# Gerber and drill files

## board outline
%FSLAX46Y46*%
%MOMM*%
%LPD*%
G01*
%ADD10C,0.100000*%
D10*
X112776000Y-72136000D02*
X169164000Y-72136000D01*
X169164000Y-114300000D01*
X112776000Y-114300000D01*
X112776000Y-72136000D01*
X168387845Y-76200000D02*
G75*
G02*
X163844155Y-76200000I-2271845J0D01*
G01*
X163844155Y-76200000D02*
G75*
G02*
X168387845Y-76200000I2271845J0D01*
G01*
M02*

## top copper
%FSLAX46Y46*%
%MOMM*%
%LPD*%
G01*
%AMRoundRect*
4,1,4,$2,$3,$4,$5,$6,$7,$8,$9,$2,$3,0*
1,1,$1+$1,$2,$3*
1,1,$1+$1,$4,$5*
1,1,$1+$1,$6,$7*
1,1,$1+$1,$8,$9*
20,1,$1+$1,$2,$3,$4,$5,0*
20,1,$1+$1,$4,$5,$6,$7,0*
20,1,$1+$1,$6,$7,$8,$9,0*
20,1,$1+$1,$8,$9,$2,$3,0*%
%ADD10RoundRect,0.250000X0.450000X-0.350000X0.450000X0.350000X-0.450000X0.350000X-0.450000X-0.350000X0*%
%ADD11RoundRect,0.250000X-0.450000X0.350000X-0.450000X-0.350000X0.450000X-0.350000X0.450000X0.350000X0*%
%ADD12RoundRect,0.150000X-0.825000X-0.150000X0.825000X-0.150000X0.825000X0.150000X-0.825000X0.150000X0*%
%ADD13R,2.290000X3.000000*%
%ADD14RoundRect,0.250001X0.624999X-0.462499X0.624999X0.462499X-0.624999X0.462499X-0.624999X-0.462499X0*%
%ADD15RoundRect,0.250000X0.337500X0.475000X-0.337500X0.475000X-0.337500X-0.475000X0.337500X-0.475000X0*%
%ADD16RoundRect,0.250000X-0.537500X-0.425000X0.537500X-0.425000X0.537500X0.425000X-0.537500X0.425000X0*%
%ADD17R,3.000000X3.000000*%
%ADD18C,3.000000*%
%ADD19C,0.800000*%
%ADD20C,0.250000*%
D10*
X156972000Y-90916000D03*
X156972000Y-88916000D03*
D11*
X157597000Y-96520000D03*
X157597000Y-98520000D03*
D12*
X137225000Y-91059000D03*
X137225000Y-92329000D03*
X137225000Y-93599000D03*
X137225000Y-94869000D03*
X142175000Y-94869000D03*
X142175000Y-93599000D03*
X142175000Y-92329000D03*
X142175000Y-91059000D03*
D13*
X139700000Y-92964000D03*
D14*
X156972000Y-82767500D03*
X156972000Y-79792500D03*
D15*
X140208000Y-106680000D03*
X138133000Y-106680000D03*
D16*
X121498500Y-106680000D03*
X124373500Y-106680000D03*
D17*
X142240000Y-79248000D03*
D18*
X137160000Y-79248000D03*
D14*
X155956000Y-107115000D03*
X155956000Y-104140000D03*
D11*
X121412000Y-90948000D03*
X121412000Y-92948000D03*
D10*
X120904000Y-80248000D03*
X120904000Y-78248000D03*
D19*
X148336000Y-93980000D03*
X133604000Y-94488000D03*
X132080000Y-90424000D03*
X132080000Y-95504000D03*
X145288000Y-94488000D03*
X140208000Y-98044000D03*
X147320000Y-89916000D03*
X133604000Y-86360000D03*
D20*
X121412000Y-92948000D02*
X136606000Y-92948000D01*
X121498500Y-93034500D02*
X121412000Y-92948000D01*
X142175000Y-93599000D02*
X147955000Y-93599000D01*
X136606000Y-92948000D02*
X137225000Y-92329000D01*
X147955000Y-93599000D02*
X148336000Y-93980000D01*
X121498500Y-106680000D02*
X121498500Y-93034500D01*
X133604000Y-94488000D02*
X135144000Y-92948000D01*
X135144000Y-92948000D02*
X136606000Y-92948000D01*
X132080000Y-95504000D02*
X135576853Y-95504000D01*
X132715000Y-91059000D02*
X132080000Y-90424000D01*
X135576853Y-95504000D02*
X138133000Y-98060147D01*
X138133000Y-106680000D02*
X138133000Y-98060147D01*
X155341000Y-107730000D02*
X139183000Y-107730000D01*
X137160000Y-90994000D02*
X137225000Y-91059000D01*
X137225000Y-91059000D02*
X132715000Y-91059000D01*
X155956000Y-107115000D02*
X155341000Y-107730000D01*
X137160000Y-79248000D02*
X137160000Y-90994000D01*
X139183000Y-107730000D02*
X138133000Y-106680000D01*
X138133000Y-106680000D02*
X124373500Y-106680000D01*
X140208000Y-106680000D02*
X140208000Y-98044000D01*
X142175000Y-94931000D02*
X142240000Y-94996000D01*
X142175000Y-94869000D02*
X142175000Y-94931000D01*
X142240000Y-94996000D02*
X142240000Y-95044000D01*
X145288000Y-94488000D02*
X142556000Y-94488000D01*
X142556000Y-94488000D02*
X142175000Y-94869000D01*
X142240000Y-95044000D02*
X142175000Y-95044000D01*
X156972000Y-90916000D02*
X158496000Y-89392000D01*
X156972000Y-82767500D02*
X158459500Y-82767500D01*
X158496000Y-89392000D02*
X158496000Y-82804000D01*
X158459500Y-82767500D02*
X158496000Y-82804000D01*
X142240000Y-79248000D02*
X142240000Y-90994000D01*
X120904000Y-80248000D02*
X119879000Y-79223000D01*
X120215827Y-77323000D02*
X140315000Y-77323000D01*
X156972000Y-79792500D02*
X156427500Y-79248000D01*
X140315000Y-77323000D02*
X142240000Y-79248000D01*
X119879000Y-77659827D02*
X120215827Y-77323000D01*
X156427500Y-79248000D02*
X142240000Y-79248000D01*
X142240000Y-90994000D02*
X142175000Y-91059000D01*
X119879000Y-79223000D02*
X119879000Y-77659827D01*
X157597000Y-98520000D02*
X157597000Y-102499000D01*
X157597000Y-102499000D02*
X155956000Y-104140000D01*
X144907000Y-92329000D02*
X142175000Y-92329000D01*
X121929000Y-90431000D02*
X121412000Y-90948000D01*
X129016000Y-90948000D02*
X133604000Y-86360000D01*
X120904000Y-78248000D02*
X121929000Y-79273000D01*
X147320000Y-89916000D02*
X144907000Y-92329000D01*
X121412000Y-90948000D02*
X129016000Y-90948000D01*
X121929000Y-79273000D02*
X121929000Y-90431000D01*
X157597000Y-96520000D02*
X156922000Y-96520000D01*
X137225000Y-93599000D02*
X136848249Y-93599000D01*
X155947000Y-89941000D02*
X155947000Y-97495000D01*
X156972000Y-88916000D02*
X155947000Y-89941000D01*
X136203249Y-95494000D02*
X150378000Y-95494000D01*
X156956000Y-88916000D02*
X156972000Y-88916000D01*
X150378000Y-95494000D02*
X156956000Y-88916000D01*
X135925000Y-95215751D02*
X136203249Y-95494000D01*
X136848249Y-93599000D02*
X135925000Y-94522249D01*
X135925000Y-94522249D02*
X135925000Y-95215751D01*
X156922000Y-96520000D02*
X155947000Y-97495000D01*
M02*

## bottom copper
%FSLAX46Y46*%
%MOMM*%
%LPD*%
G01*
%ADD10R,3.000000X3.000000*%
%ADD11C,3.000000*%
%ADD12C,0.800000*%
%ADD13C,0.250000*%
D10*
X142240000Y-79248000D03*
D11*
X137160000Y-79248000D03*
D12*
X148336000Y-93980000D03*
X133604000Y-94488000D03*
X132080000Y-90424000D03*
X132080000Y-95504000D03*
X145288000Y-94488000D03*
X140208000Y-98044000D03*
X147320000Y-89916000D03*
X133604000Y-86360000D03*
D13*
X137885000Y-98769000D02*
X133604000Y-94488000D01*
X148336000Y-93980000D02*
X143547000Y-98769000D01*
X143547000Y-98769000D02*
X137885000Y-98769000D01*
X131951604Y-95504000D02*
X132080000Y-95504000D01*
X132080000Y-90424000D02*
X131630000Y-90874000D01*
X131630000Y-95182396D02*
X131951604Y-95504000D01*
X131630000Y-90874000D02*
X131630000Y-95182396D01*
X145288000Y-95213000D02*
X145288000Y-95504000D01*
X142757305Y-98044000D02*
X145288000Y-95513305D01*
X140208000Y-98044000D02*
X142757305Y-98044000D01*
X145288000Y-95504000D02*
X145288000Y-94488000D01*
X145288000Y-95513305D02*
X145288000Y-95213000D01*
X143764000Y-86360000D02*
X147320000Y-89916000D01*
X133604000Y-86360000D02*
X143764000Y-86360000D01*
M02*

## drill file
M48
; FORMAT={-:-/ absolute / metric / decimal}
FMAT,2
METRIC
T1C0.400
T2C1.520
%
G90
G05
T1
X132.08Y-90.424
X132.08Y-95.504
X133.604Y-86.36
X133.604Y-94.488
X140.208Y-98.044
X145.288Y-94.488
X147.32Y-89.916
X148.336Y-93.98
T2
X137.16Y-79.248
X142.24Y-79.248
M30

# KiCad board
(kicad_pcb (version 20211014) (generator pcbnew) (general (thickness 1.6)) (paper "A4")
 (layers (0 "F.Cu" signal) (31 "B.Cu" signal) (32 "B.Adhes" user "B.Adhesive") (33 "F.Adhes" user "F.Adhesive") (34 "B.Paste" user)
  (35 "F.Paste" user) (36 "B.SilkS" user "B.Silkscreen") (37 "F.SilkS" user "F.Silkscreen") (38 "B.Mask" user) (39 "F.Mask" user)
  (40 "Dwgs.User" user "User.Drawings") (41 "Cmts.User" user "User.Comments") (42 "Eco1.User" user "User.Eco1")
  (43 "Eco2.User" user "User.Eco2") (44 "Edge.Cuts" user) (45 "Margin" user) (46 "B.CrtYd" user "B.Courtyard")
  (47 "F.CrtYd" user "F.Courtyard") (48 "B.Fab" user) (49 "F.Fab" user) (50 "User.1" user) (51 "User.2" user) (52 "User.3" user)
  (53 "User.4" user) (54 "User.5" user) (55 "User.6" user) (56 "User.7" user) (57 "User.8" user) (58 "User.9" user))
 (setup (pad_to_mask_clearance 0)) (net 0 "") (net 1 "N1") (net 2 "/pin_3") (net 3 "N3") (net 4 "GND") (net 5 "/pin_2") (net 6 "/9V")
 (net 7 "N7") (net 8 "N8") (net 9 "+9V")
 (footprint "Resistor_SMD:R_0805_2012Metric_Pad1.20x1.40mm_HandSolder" (layer "F.Cu") (at 156.972 89.916 90)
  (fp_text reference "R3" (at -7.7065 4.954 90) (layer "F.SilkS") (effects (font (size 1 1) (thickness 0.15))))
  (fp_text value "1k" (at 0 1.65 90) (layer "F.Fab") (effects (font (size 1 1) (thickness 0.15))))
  (pad "1" smd roundrect (at -1 0 90) (size 1.2 1.4) (layers "F.Cu" "F.Paste" "F.Mask") (roundrect_rratio 0.208333) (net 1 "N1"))
  (pad "2" smd roundrect (at 1 0 90) (size 1.2 1.4) (layers "F.Cu" "F.Paste" "F.Mask") (roundrect_rratio 0.208333) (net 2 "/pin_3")))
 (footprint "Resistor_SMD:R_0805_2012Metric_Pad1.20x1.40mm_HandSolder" (layer "F.Cu") (at 157.597 97.52 -90)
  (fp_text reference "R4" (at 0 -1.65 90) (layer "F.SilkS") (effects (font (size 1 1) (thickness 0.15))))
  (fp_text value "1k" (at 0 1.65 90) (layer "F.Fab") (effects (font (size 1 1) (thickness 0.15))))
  (pad "1" smd roundrect (at -1 0 270) (size 1.2 1.4) (layers "F.Cu" "F.Paste" "F.Mask") (roundrect_rratio 0.208333) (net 2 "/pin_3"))
  (pad "2" smd roundrect (at 1 0 270) (size 1.2 1.4) (layers "F.Cu" "F.Paste" "F.Mask") (roundrect_rratio 0.208333) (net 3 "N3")))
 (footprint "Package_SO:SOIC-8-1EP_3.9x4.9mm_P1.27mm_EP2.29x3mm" (layer "F.Cu") (at 139.7 92.964)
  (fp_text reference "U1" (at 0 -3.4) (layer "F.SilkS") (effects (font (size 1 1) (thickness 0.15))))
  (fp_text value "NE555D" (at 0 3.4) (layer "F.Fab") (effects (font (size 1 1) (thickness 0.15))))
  (pad "" smd roundrect (at 0.57 -0.75) (size 0.92 1.21) (layers "F.Paste") (roundrect_rratio 0.25))
  (pad "" smd roundrect (at -0.57 0.75) (size 0.92 1.21) (layers "F.Paste") (roundrect_rratio 0.25))
  (pad "" smd roundrect (at -0.57 -0.75) (size 0.92 1.21) (layers "F.Paste") (roundrect_rratio 0.25))
  (pad "" smd roundrect (at 0.57 0.75) (size 0.92 1.21) (layers "F.Paste") (roundrect_rratio 0.25))
  (pad "1" smd roundrect (at -2.475 -1.905) (size 1.95 0.6) (layers "F.Cu" "F.Paste" "F.Mask") (roundrect_rratio 0.25) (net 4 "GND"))
  (pad "2" smd roundrect (at -2.475 -0.635) (size 1.95 0.6) (layers "F.Cu" "F.Paste" "F.Mask") (roundrect_rratio 0.25) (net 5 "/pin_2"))
  (pad "3" smd roundrect (at -2.475 0.635) (size 1.95 0.6) (layers "F.Cu" "F.Paste" "F.Mask") (roundrect_rratio 0.25) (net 2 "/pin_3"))
  (pad "4" smd roundrect (at -2.475 1.905) (size 1.95 0.6) (layers "F.Cu" "F.Paste" "F.Mask") (roundrect_rratio 0.25) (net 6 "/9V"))
  (pad "5" smd roundrect (at 2.475 1.905) (size 1.95 0.6) (layers "F.Cu" "F.Paste" "F.Mask") (roundrect_rratio 0.25) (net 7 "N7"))
  (pad "6" smd roundrect (at 2.475 0.635) (size 1.95 0.6) (layers "F.Cu" "F.Paste" "F.Mask") (roundrect_rratio 0.25) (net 5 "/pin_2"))
  (pad "7" smd roundrect (at 2.475 -0.635) (size 1.95 0.6) (layers "F.Cu" "F.Paste" "F.Mask") (roundrect_rratio 0.25) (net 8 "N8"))
  (pad "8" smd roundrect (at 2.475 -1.905) (size 1.95 0.6) (layers "F.Cu" "F.Paste" "F.Mask") (roundrect_rratio 0.25) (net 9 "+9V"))
  (pad "9" smd rect (at 0 0) (size 2.29 3) (layers "F.Cu" "F.Mask")))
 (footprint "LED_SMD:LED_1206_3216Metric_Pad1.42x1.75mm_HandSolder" (layer "F.Cu") (at 156.972 81.28 90)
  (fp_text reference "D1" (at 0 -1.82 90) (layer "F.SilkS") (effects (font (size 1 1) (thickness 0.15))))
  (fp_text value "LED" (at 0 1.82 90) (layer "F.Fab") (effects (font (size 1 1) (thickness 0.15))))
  (pad "1" smd roundrect (at -1.4875 0 90) (size 1.425 1.75) (layers "F.Cu" "F.Paste" "F.Mask") (roundrect_rratio 0.175439) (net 1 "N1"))
  (pad "2" smd roundrect (at 1.4875 0 90) (size 1.425 1.75) (layers "F.Cu" "F.Paste" "F.Mask") (roundrect_rratio 0.175439) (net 9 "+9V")))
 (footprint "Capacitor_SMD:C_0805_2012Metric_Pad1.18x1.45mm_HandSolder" (layer "F.Cu") (at 139.1705 106.68 180)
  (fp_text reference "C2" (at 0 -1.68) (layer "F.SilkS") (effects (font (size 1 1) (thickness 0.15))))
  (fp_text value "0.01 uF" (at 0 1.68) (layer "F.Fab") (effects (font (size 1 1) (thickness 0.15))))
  (pad "1" smd roundrect (at -1.0375 0 180) (size 1.175 1.45) (layers "F.Cu" "F.Paste" "F.Mask") (roundrect_rratio 0.212766) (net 7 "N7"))
  (pad "2" smd roundrect (at 1.0375 0 180) (size 1.175 1.45) (layers "F.Cu" "F.Paste" "F.Mask") (roundrect_rratio 0.212766) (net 4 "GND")))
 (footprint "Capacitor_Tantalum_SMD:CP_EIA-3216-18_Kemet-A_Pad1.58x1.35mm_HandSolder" (layer "F.Cu") (at 122.936 106.68)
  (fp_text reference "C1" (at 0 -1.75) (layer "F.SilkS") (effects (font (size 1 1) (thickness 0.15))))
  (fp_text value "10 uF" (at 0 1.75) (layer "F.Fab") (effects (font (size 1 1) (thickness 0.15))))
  (pad "1" smd roundrect (at -1.4375 0) (size 1.575 1.35) (layers "F.Cu" "F.Paste" "F.Mask") (roundrect_rratio 0.185185) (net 5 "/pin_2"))
  (pad "2" smd roundrect (at 1.4375 0) (size 1.575 1.35) (layers "F.Cu" "F.Paste" "F.Mask") (roundrect_rratio 0.185185) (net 4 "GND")))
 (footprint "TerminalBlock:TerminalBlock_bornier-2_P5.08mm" (layer "F.Cu") (at 142.24 79.248 180)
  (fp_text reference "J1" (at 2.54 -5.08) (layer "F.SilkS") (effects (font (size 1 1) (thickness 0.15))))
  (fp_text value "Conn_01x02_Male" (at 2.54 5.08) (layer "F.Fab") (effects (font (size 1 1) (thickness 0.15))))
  (pad "1" thru_hole rect (at 0 0 180) (size 3 3) (drill 1.52) (layers *.Cu *.Mask) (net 9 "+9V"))
  (pad "2" thru_hole circle (at 5.08 0 180) (size 3 3) (drill 1.52) (layers *.Cu *.Mask) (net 4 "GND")))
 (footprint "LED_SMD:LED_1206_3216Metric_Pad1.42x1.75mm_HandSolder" (layer "F.Cu") (at 155.956 105.6275 90)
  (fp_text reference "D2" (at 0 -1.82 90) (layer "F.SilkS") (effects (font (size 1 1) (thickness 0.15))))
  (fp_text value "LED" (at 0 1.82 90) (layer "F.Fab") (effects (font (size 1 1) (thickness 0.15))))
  (pad "1" smd roundrect (at -1.4875 0 90) (size 1.425 1.75) (layers "F.Cu" "F.Paste" "F.Mask") (roundrect_rratio 0.175439) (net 4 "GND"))
  (pad "2" smd roundrect (at 1.4875 0 90) (size 1.425 1.75) (layers "F.Cu" "F.Paste" "F.Mask") (roundrect_rratio 0.175439) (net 3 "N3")))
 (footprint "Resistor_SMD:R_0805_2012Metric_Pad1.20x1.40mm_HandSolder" (layer "F.Cu") (at 121.412 91.948 -90)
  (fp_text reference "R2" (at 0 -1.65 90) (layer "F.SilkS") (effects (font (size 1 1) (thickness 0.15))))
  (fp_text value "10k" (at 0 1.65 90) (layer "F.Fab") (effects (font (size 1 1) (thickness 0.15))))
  (pad "1" smd roundrect (at -1 0 270) (size 1.2 1.4) (layers "F.Cu" "F.Paste" "F.Mask") (roundrect_rratio 0.208333) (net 8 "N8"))
  (pad "2" smd roundrect (at 1 0 270) (size 1.2 1.4) (layers "F.Cu" "F.Paste" "F.Mask") (roundrect_rratio 0.208333) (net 5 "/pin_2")))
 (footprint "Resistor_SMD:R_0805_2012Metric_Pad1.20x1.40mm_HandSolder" (layer "F.Cu") (at 120.904 79.248 90)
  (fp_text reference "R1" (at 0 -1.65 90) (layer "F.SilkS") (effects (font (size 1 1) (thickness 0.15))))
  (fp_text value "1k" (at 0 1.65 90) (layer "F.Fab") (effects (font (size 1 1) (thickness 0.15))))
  (pad "1" smd roundrect (at -1 0 90) (size 1.2 1.4) (layers "F.Cu" "F.Paste" "F.Mask") (roundrect_rratio 0.208333) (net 9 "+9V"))
  (pad "2" smd roundrect (at 1 0 90) (size 1.2 1.4) (layers "F.Cu" "F.Paste" "F.Mask") (roundrect_rratio 0.208333) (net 8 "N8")))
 (gr_rect (start 112.776 72.136) (end 169.164 114.3) (layer "Edge.Cuts") (width 0.1) (fill none))
 (gr_circle (center 166.116 76.2) (end 164.084 75.184) (layer "Edge.Cuts") (width 0.1) (fill none))
 (segment (start 121.412 92.948) (end 136.606 92.948) (width 0.25) (layer "F.Cu") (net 5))
 (segment (start 121.4985 93.0345) (end 121.412 92.948) (width 0.25) (layer "F.Cu") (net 5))
 (segment (start 142.175 93.599) (end 147.955 93.599) (width 0.25) (layer "F.Cu") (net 5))
 (segment (start 136.606 92.948) (end 137.225 92.329) (width 0.25) (layer "F.Cu") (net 5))
 (segment (start 147.955 93.599) (end 148.336 93.98) (width 0.25) (layer "F.Cu") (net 5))
 (segment (start 121.4985 106.68) (end 121.4985 93.0345) (width 0.25) (layer "F.Cu") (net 5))
 (segment (start 133.604 94.488) (end 135.144 92.948) (width 0.25) (layer "F.Cu") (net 5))
 (segment (start 135.144 92.948) (end 136.606 92.948) (width 0.25) (layer "F.Cu") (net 5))
 (via (at 148.336 93.98) (size 0.8) (drill 0.4) (layers "F.Cu" "B.Cu") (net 5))
 (via (at 133.604 94.488) (size 0.8) (drill 0.4) (layers "F.Cu" "B.Cu") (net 5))
 (segment (start 137.885 98.769) (end 133.604 94.488) (width 0.25) (layer "B.Cu") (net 5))
 (segment (start 148.336 93.98) (end 143.547 98.769) (width 0.25) (layer "B.Cu") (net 5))
 (segment (start 143.547 98.769) (end 137.885 98.769) (width 0.25) (layer "B.Cu") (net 5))
 (segment (start 132.08 95.504) (end 135.576853 95.504) (width 0.25) (layer "F.Cu") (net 4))
 (segment (start 132.715 91.059) (end 132.08 90.424) (width 0.25) (layer "F.Cu") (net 4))
 (segment (start 135.576853 95.504) (end 138.133 98.060147) (width 0.25) (layer "F.Cu") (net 4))
 (segment (start 138.133 106.68) (end 138.133 98.060147) (width 0.25) (layer "F.Cu") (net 4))
 (segment (start 155.341 107.73) (end 139.183 107.73) (width 0.25) (layer "F.Cu") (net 4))
 (segment (start 137.16 90.994) (end 137.225 91.059) (width 0.25) (layer "F.Cu") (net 4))
 (segment (start 137.225 91.059) (end 132.715 91.059) (width 0.25) (layer "F.Cu") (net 4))
 (segment (start 155.956 107.115) (end 155.341 107.73) (width 0.25) (layer "F.Cu") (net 4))
 (segment (start 137.16 79.248) (end 137.16 90.994) (width 0.25) (layer "F.Cu") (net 4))
 (segment (start 139.183 107.73) (end 138.133 106.68) (width 0.25) (layer "F.Cu") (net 4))
 (segment (start 138.133 106.68) (end 124.3735 106.68) (width 0.25) (layer "F.Cu") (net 4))
 (via (at 132.08 90.424) (size 0.8) (drill 0.4) (layers "F.Cu" "B.Cu") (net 4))
 (via (at 132.08 95.504) (size 0.8) (drill 0.4) (layers "F.Cu" "B.Cu") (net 4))
 (segment (start 131.951604 95.504) (end 132.08 95.504) (width 0.25) (layer "B.Cu") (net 4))
 (segment (start 132.08 90.424) (end 131.63 90.874) (width 0.25) (layer "B.Cu") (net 4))
 (segment (start 131.63 95.182396) (end 131.951604 95.504) (width 0.25) (layer "B.Cu") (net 4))
 (segment (start 131.63 90.874) (end 131.63 95.182396) (width 0.25) (layer "B.Cu") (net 4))
 (segment (start 140.208 106.68) (end 140.208 98.044) (width 0.25) (layer "F.Cu") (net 7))
 (segment (start 142.175 94.931) (end 142.24 94.996) (width 0.25) (layer "F.Cu") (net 7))
 (segment (start 142.175 94.869) (end 142.175 94.931) (width 0.25) (layer "F.Cu") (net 7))
 (segment (start 142.24 94.996) (end 142.24 95.044) (width 0.25) (layer "F.Cu") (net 7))
 (segment (start 145.288 94.488) (end 142.556 94.488) (width 0.25) (layer "F.Cu") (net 7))
 (segment (start 142.556 94.488) (end 142.175 94.869) (width 0.25) (layer "F.Cu") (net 7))
 (segment (start 142.24 95.044) (end 142.175 95.044) (width 0.25) (layer "F.Cu") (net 7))
 (via (at 145.288 94.488) (size 0.8) (drill 0.4) (layers "F.Cu" "B.Cu") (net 7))
 (via (at 140.208 98.044) (size 0.8) (drill 0.4) (layers "F.Cu" "B.Cu") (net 7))
 (segment (start 145.288 95.213) (end 145.288 95.504) (width 0.25) (layer "B.Cu") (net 7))
 (segment (start 142.757305 98.044) (end 145.288 95.513305) (width 0.25) (layer "B.Cu") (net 7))
 (segment (start 140.208 98.044) (end 142.757305 98.044) (width 0.25) (layer "B.Cu") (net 7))
 (segment (start 145.288 95.504) (end 145.288 94.488) (width 0.25) (layer "B.Cu") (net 7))
 (segment (start 145.288 95.513305) (end 145.288 95.213) (width 0.25) (layer "B.Cu") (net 7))
 (segment (start 156.972 90.916) (end 158.496 89.392) (width 0.25) (layer "F.Cu") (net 1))
 (segment (start 156.972 82.7675) (end 158.4595 82.7675) (width 0.25) (layer "F.Cu") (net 1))
 (segment (start 158.496 89.392) (end 158.496 82.804) (width 0.25) (layer "F.Cu") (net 1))
 (segment (start 158.4595 82.7675) (end 158.496 82.804) (width 0.25) (layer "F.Cu") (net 1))
 (segment (start 142.24 79.248) (end 142.24 90.994) (width 0.25) (layer "F.Cu") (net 9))
 (segment (start 120.904 80.248) (end 119.879 79.223) (width 0.25) (layer "F.Cu") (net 9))
 (segment (start 120.215827 77.323) (end 140.315 77.323) (width 0.25) (layer "F.Cu") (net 9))
 (segment (start 156.972 79.7925) (end 156.4275 79.248) (width 0.25) (layer "F.Cu") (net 9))
 (segment (start 140.315 77.323) (end 142.24 79.248) (width 0.25) (layer "F.Cu") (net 9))
 (segment (start 119.879 77.659827) (end 120.215827 77.323) (width 0.25) (layer "F.Cu") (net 9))
 (segment (start 156.4275 79.248) (end 142.24 79.248) (width 0.25) (layer "F.Cu") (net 9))
 (segment (start 142.24 90.994) (end 142.175 91.059) (width 0.25) (layer "F.Cu") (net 9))
 (segment (start 119.879 79.223) (end 119.879 77.659827) (width 0.25) (layer "F.Cu") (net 9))
 (segment (start 157.597 98.52) (end 157.597 102.499) (width 0.25) (layer "F.Cu") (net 3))
 (segment (start 157.597 102.499) (end 155.956 104.14) (width 0.25) (layer "F.Cu") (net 3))
 (segment (start 144.907 92.329) (end 142.175 92.329) (width 0.25) (layer "F.Cu") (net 8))
 (segment (start 121.929 90.431) (end 121.412 90.948) (width 0.25) (layer "F.Cu") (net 8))
 (segment (start 129.016 90.948) (end 133.604 86.36) (width 0.25) (layer "F.Cu") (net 8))
 (segment (start 120.904 78.248) (end 121.929 79.273) (width 0.25) (layer "F.Cu") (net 8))
 (segment (start 147.32 89.916) (end 144.907 92.329) (width 0.25) (layer "F.Cu") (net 8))
 (segment (start 121.412 90.948) (end 129.016 90.948) (width 0.25) (layer "F.Cu") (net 8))
 (segment (start 121.929 79.273) (end 121.929 90.431) (width 0.25) (layer "F.Cu") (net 8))
 (via (at 147.32 89.916) (size 0.8) (drill 0.4) (layers "F.Cu" "B.Cu") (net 8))
 (via (at 133.604 86.36) (size 0.8) (drill 0.4) (layers "F.Cu" "B.Cu") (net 8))
 (segment (start 143.764 86.36) (end 147.32 89.916) (width 0.25) (layer "B.Cu") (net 8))
 (segment (start 133.604 86.36) (end 143.764 86.36) (width 0.25) (layer "B.Cu") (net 8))
 (segment (start 157.597 96.52) (end 156.922 96.52) (width 0.25) (layer "F.Cu") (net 2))
 (segment (start 137.225 93.599) (end 136.848249 93.599) (width 0.25) (layer "F.Cu") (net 2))
 (segment (start 155.947 89.941) (end 155.947 97.495) (width 0.25) (layer "F.Cu") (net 2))
 (segment (start 156.972 88.916) (end 155.947 89.941) (width 0.25) (layer "F.Cu") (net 2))
 (segment (start 136.203249 95.494) (end 150.378 95.494) (width 0.25) (layer "F.Cu") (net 2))
 (segment (start 156.956 88.916) (end 156.972 88.916) (width 0.25) (layer "F.Cu") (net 2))
 (segment (start 150.378 95.494) (end 156.956 88.916) (width 0.25) (layer "F.Cu") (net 2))
 (segment (start 135.925 95.215751) (end 136.203249 95.494) (width 0.25) (layer "F.Cu") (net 2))
 (segment (start 136.848249 93.599) (end 135.925 94.522249) (width 0.25) (layer "F.Cu") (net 2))
 (segment (start 135.925 94.522249) (end 135.925 95.215751) (width 0.25) (layer "F.Cu") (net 2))
 (segment (start 156.922 96.52) (end 155.947 97.495) (width 0.25) (layer "F.Cu") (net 2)))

